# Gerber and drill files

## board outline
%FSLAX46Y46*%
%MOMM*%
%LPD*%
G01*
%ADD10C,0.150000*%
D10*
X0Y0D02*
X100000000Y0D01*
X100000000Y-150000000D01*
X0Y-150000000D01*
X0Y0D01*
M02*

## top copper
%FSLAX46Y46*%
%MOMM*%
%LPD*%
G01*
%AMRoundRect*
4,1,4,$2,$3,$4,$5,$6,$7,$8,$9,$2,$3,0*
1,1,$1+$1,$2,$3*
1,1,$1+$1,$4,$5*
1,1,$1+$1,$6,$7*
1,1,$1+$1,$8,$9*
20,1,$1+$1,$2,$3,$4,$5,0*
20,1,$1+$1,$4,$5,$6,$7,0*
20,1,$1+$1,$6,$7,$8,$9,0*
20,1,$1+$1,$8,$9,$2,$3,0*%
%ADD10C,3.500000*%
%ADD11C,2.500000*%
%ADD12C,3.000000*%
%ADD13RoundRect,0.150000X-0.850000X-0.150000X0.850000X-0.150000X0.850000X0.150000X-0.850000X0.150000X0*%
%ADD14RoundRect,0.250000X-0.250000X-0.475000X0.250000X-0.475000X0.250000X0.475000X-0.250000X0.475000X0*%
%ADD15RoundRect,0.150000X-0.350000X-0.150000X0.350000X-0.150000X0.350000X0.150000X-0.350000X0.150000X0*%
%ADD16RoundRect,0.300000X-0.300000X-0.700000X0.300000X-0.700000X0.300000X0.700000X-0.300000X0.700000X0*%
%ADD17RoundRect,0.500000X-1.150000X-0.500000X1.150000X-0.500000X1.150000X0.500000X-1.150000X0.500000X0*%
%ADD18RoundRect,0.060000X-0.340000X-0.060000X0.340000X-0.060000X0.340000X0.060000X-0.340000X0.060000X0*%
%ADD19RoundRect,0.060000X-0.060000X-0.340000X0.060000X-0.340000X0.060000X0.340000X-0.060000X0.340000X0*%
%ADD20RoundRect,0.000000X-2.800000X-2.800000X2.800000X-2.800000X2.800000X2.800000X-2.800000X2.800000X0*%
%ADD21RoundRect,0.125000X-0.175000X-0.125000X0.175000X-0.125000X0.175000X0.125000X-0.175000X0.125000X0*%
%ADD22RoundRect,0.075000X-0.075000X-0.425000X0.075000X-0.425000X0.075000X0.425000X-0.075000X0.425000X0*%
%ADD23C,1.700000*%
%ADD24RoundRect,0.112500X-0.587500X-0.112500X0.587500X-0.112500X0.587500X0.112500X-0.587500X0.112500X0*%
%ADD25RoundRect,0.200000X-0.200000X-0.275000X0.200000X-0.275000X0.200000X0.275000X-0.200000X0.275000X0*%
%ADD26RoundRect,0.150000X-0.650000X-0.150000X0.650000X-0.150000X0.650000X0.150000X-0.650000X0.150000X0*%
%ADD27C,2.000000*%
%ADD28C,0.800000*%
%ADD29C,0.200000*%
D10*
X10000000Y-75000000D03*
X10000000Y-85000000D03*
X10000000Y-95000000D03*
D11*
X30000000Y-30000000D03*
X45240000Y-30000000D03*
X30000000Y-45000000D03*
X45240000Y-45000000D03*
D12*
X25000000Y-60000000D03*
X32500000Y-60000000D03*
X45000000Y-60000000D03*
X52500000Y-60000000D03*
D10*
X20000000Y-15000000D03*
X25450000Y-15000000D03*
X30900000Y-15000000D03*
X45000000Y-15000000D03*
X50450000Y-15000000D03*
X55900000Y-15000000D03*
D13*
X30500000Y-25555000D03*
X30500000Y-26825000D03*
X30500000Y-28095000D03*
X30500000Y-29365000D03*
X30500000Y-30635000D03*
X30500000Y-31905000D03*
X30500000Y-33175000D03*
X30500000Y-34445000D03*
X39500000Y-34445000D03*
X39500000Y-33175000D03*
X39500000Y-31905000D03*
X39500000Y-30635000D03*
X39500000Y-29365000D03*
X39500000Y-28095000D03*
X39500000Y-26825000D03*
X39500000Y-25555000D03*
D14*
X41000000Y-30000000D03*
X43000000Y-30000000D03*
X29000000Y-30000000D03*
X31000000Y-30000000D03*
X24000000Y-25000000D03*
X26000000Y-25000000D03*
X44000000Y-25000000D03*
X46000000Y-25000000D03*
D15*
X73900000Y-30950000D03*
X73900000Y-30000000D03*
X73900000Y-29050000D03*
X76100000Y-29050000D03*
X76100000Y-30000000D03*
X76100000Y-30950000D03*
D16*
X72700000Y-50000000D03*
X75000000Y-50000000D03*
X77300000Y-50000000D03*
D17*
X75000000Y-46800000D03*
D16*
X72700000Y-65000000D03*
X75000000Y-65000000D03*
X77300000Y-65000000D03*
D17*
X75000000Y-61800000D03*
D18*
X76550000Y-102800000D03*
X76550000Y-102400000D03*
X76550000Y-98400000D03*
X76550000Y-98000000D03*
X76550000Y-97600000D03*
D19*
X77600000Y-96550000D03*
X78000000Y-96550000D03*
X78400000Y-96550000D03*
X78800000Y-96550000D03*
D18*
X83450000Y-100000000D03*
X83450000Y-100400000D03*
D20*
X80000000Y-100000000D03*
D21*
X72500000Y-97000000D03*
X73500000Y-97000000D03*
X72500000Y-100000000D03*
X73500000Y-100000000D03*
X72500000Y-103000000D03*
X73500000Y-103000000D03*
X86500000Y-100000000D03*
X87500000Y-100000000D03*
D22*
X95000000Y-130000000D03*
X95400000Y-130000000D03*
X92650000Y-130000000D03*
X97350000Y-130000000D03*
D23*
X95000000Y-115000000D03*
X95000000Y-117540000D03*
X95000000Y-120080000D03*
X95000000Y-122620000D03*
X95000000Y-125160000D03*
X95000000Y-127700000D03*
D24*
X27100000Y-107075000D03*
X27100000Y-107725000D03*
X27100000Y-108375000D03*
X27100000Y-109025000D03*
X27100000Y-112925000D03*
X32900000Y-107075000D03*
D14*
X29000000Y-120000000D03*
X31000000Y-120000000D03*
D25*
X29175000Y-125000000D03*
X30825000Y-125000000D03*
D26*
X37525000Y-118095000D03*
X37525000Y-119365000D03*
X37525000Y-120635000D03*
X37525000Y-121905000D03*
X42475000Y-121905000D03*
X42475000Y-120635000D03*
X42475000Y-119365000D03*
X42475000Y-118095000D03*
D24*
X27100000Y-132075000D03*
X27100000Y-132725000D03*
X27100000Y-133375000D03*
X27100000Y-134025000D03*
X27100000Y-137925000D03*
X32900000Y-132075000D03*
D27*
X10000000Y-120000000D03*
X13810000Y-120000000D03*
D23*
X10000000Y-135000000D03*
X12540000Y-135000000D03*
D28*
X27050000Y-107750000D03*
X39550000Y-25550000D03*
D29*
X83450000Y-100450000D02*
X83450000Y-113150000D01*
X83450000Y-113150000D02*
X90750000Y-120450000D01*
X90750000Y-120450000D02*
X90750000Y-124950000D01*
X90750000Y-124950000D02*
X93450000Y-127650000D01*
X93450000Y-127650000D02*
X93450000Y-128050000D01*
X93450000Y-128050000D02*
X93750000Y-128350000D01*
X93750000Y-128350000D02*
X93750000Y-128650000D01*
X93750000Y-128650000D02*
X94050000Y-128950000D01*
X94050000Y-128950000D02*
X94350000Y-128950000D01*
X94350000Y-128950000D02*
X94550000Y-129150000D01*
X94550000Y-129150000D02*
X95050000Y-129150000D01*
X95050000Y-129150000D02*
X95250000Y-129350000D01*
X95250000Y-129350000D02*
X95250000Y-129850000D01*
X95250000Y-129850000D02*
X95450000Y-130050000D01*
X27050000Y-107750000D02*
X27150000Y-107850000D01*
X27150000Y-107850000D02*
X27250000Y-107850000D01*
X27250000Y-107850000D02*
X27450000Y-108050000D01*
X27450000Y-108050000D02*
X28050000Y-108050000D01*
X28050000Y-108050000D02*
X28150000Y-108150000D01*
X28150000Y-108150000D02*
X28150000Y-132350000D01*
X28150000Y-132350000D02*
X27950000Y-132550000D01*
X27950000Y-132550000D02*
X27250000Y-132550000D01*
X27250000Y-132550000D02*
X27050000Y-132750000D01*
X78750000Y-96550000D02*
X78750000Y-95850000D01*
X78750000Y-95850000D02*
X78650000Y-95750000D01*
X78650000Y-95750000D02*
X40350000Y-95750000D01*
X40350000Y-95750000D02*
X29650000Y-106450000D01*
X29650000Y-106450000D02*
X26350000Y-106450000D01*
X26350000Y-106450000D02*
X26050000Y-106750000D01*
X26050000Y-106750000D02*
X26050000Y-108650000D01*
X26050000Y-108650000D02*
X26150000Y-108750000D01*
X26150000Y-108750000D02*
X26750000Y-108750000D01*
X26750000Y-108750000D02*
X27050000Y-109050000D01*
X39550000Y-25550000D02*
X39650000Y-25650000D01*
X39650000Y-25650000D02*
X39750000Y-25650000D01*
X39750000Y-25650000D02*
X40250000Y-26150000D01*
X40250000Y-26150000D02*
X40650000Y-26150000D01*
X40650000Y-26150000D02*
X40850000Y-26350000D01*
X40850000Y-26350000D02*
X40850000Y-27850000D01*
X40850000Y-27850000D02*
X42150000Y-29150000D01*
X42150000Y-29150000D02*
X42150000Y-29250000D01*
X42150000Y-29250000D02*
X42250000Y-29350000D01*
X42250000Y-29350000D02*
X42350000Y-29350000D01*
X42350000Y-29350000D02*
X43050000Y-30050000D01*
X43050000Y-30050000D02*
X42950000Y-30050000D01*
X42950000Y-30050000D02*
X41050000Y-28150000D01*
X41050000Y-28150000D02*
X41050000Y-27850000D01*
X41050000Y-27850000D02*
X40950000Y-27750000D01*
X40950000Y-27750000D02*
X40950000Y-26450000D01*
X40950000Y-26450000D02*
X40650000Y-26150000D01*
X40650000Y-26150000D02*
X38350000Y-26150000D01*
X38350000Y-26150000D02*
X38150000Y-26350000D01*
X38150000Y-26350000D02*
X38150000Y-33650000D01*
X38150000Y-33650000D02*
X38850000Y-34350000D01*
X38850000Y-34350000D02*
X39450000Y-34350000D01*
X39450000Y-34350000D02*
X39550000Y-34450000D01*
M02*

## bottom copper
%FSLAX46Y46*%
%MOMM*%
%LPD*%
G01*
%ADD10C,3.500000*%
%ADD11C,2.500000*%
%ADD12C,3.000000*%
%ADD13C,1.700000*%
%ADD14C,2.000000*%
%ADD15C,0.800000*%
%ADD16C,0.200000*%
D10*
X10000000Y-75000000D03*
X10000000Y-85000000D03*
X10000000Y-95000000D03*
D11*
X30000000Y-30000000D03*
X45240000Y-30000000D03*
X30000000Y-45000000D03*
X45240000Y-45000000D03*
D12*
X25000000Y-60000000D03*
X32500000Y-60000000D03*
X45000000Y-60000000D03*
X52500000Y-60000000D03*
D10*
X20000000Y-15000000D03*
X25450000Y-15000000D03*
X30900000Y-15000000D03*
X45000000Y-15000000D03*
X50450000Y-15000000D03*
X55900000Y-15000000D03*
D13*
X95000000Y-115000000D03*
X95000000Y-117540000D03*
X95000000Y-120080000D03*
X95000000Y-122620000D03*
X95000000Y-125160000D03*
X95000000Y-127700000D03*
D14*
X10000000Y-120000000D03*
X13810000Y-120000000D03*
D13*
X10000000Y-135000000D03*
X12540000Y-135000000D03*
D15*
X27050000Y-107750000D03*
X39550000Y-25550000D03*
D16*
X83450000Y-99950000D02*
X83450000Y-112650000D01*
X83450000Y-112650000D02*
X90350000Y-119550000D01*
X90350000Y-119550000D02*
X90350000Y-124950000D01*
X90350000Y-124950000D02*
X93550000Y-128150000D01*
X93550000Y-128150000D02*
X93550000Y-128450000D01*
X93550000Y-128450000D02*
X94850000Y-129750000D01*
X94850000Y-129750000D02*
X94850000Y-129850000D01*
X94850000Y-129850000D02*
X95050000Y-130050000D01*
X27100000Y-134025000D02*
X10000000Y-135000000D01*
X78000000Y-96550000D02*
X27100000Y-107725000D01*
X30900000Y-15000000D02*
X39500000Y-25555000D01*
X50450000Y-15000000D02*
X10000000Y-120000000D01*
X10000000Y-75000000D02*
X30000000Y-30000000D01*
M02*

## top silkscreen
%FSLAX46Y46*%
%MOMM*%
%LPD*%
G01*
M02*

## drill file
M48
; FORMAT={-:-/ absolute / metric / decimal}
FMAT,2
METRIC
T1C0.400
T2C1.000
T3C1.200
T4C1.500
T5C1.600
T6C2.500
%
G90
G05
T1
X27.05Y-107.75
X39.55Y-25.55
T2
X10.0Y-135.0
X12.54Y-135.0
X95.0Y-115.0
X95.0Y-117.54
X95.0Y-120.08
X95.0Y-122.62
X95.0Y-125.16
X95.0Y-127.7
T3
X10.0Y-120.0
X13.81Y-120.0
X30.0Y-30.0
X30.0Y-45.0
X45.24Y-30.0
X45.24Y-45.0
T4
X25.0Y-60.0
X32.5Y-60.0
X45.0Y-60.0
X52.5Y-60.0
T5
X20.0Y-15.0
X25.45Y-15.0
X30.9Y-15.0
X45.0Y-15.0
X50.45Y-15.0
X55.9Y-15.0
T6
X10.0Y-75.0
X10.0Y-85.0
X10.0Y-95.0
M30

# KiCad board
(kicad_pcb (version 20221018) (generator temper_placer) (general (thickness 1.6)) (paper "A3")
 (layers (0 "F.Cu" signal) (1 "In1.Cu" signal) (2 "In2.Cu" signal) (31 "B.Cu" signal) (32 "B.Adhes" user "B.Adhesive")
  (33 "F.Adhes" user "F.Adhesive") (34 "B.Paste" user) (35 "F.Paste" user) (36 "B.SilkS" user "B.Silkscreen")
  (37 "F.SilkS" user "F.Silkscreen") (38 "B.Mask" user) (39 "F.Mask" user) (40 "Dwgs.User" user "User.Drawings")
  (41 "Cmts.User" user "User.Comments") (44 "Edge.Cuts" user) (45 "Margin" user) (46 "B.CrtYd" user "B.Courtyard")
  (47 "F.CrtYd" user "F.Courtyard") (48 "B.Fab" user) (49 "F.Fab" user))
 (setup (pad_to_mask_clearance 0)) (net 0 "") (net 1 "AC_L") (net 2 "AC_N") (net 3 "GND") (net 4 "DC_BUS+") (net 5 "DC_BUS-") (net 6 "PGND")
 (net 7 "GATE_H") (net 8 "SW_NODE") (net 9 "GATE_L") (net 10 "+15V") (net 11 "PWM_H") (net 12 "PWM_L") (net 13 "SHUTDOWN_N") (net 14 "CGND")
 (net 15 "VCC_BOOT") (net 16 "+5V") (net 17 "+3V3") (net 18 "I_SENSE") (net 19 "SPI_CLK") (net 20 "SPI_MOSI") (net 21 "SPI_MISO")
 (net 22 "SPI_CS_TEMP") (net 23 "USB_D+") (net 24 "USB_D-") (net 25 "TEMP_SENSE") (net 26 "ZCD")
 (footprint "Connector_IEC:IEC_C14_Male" (layer "F.Cu") (at 10 75) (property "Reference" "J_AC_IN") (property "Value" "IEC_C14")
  (pad "1" thru_hole circle (at 0 0) (size 3.5 3.5) (drill 2.5) (layers *.Cu *.Mask) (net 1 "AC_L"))
  (pad "2" thru_hole circle (at 0 10) (size 3.5 3.5) (drill 2.5) (layers *.Cu *.Mask) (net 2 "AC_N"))
  (pad "3" thru_hole circle (at 0 20) (size 3.5 3.5) (drill 2.5) (layers *.Cu *.Mask) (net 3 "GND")))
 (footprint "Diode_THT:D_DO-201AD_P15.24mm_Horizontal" (layer "F.Cu") (at 30 30) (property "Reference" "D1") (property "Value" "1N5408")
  (pad "1" thru_hole circle (at 0 0) (size 2.5 2.5) (drill 1.2) (layers *.Cu *.Mask) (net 1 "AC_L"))
  (pad "2" thru_hole circle (at 15.24 0) (size 2.5 2.5) (drill 1.2) (layers *.Cu *.Mask) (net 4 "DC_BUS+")))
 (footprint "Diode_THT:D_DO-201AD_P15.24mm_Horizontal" (layer "F.Cu") (at 30 45) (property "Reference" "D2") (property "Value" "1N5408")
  (pad "1" thru_hole circle (at 0 0) (size 2.5 2.5) (drill 1.2) (layers *.Cu *.Mask) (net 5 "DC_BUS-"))
  (pad "2" thru_hole circle (at 15.24 0) (size 2.5 2.5) (drill 1.2) (layers *.Cu *.Mask) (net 2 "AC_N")))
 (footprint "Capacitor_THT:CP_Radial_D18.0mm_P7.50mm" (layer "F.Cu") (at 25 60) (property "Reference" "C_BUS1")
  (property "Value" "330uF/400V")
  (pad "1" thru_hole circle (at 0 0) (size 3 3) (drill 1.5) (layers *.Cu *.Mask) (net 4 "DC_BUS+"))
  (pad "2" thru_hole circle (at 7.5 0) (size 3 3) (drill 1.5) (layers *.Cu *.Mask) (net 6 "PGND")))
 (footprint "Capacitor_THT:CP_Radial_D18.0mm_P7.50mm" (layer "F.Cu") (at 45 60) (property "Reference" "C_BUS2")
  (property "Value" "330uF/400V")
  (pad "1" thru_hole circle (at 0 0) (size 3 3) (drill 1.5) (layers *.Cu *.Mask) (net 6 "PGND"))
  (pad "2" thru_hole circle (at 7.5 0) (size 3 3) (drill 1.5) (layers *.Cu *.Mask) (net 5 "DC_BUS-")))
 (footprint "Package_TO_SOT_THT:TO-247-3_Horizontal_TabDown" (layer "F.Cu") (at 20 15) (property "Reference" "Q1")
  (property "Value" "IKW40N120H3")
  (pad "1" thru_hole circle (at 0 0) (size 3.5 3.5) (drill 1.6) (layers *.Cu *.Mask) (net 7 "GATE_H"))
  (pad "2" thru_hole circle (at 5.45 0) (size 3.5 3.5) (drill 1.6) (layers *.Cu *.Mask) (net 4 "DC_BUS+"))
  (pad "3" thru_hole circle (at 10.9 0) (size 3.5 3.5) (drill 1.6) (layers *.Cu *.Mask) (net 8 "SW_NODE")))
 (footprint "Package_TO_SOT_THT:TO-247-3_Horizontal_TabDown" (layer "F.Cu") (at 45 15) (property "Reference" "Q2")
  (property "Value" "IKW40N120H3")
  (pad "1" thru_hole circle (at 0 0) (size 3.5 3.5) (drill 1.6) (layers *.Cu *.Mask) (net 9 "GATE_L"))
  (pad "2" thru_hole circle (at 5.45 0) (size 3.5 3.5) (drill 1.6) (layers *.Cu *.Mask) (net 8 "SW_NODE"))
  (pad "3" thru_hole circle (at 10.9 0) (size 3.5 3.5) (drill 1.6) (layers *.Cu *.Mask) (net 5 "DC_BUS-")))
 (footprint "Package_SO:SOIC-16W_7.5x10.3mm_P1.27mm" (layer "F.Cu") (at 35 30) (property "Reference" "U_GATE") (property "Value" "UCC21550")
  (pad "1" smd roundrect (at -4.5 -4.445) (size 2 0.6) (layers "F.Cu" "F.Paste" "F.Mask") (roundrect_rratio 0.25) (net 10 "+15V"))
  (pad "2" smd roundrect (at -4.5 -3.175) (size 2 0.6) (layers "F.Cu" "F.Paste" "F.Mask") (roundrect_rratio 0.25) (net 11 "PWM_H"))
  (pad "3" smd roundrect (at -4.5 -1.905) (size 2 0.6) (layers "F.Cu" "F.Paste" "F.Mask") (roundrect_rratio 0.25) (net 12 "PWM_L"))
  (pad "4" smd roundrect (at -4.5 -0.635) (size 2 0.6) (layers "F.Cu" "F.Paste" "F.Mask") (roundrect_rratio 0.25) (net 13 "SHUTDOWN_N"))
  (pad "5" smd roundrect (at -4.5 0.635) (size 2 0.6) (layers "F.Cu" "F.Paste" "F.Mask") (roundrect_rratio 0.25) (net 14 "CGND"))
  (pad "6" smd roundrect (at -4.5 1.905) (size 2 0.6) (layers "F.Cu" "F.Paste" "F.Mask") (roundrect_rratio 0.25) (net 14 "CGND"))
  (pad "7" smd roundrect (at -4.5 3.175) (size 2 0.6) (layers "F.Cu" "F.Paste" "F.Mask") (roundrect_rratio 0.25) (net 14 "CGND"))
  (pad "8" smd roundrect (at -4.5 4.445) (size 2 0.6) (layers "F.Cu" "F.Paste" "F.Mask") (roundrect_rratio 0.25) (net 14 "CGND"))
  (pad "9" smd roundrect (at 4.5 4.445) (size 2 0.6) (layers "F.Cu" "F.Paste" "F.Mask") (roundrect_rratio 0.25) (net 8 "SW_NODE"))
  (pad "10" smd roundrect (at 4.5 3.175) (size 2 0.6) (layers "F.Cu" "F.Paste" "F.Mask") (roundrect_rratio 0.25) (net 9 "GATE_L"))
  (pad "11" smd roundrect (at 4.5 1.905) (size 2 0.6) (layers "F.Cu" "F.Paste" "F.Mask") (roundrect_rratio 0.25) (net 10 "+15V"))
  (pad "12" smd roundrect (at 4.5 0.635) (size 2 0.6) (layers "F.Cu" "F.Paste" "F.Mask") (roundrect_rratio 0.25) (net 6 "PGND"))
  (pad "13" smd roundrect (at 4.5 -0.635) (size 2 0.6) (layers "F.Cu" "F.Paste" "F.Mask") (roundrect_rratio 0.25) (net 6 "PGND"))
  (pad "14" smd roundrect (at 4.5 -1.905) (size 2 0.6) (layers "F.Cu" "F.Paste" "F.Mask") (roundrect_rratio 0.25) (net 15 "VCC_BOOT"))
  (pad "15" smd roundrect (at 4.5 -3.175) (size 2 0.6) (layers "F.Cu" "F.Paste" "F.Mask") (roundrect_rratio 0.25) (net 7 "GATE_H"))
  (pad "16" smd roundrect (at 4.5 -4.445) (size 2 0.6) (layers "F.Cu" "F.Paste" "F.Mask") (roundrect_rratio 0.25) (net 8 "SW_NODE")))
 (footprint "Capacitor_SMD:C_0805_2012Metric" (layer "F.Cu") (at 42 30) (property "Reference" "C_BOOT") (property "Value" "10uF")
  (pad "1" smd roundrect (at -1 0) (size 1 1.45) (layers "F.Cu" "F.Paste" "F.Mask") (roundrect_rratio 0.25) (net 15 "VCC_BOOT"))
  (pad "2" smd roundrect (at 1 0) (size 1 1.45) (layers "F.Cu" "F.Paste" "F.Mask") (roundrect_rratio 0.25) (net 8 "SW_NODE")))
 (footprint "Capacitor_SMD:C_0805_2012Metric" (layer "F.Cu") (at 30 30) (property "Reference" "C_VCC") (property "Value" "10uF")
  (pad "1" smd roundrect (at -1 0) (size 1 1.45) (layers "F.Cu" "F.Paste" "F.Mask") (roundrect_rratio 0.25) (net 10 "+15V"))
  (pad "2" smd roundrect (at 1 0) (size 1 1.45) (layers "F.Cu" "F.Paste" "F.Mask") (roundrect_rratio 0.25) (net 14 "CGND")))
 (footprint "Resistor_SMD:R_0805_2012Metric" (layer "F.Cu") (at 25 25) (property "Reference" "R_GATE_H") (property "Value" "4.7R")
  (pad "1" smd roundrect (at -1 0) (size 1 1.45) (layers "F.Cu" "F.Paste" "F.Mask") (roundrect_rratio 0.25) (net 7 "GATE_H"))
  (pad "2" smd roundrect (at 1 0) (size 1 1.45) (layers "F.Cu" "F.Paste" "F.Mask") (roundrect_rratio 0.25) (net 7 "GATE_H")))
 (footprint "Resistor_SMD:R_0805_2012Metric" (layer "F.Cu") (at 45 25) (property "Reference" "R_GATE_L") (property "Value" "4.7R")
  (pad "1" smd roundrect (at -1 0) (size 1 1.45) (layers "F.Cu" "F.Paste" "F.Mask") (roundrect_rratio 0.25) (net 9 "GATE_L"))
  (pad "2" smd roundrect (at 1 0) (size 1 1.45) (layers "F.Cu" "F.Paste" "F.Mask") (roundrect_rratio 0.25) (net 9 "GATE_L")))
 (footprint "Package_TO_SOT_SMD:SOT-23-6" (layer "F.Cu") (at 75 30) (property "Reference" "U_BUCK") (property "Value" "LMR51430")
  (pad "1" smd roundrect (at -1.1 0.95) (size 1 0.6) (layers "F.Cu" "F.Paste" "F.Mask") (roundrect_rratio 0.25) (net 3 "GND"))
  (pad "2" smd roundrect (at -1.1 0) (size 1 0.6) (layers "F.Cu" "F.Paste" "F.Mask") (roundrect_rratio 0.25) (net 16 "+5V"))
  (pad "3" smd roundrect (at -1.1 -0.95) (size 1 0.6) (layers "F.Cu" "F.Paste" "F.Mask") (roundrect_rratio 0.25) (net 10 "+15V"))
  (pad "4" smd roundrect (at 1.1 -0.95) (size 1 0.6) (layers "F.Cu" "F.Paste" "F.Mask") (roundrect_rratio 0.25) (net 16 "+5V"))
  (pad "5" smd roundrect (at 1.1 0) (size 1 0.6) (layers "F.Cu" "F.Paste" "F.Mask") (roundrect_rratio 0.25) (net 3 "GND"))
  (pad "6" smd roundrect (at 1.1 0.95) (size 1 0.6) (layers "F.Cu" "F.Paste" "F.Mask") (roundrect_rratio 0.25) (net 3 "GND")))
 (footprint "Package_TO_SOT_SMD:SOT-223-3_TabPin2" (layer "F.Cu") (at 75 50) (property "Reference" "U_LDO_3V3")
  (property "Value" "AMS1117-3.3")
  (pad "1" smd roundrect (at -2.3 0) (size 1.2 2) (layers "F.Cu" "F.Paste" "F.Mask") (roundrect_rratio 0.25) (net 3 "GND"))
  (pad "2" smd roundrect (at 0 0) (size 1.2 2) (layers "F.Cu" "F.Paste" "F.Mask") (roundrect_rratio 0.25) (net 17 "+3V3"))
  (pad "3" smd roundrect (at 2.3 0) (size 1.2 2) (layers "F.Cu" "F.Paste" "F.Mask") (roundrect_rratio 0.25) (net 16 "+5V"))
  (pad "4" smd roundrect (at 0 -3.2) (size 3.3 2) (layers "F.Cu" "F.Paste" "F.Mask") (roundrect_rratio 0.25) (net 17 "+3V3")))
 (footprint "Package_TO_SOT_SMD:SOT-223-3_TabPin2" (layer "F.Cu") (at 75 65) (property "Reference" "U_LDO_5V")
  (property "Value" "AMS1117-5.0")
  (pad "1" smd roundrect (at -2.3 0) (size 1.2 2) (layers "F.Cu" "F.Paste" "F.Mask") (roundrect_rratio 0.25) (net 3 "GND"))
  (pad "2" smd roundrect (at 0 0) (size 1.2 2) (layers "F.Cu" "F.Paste" "F.Mask") (roundrect_rratio 0.25) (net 16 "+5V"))
  (pad "3" smd roundrect (at 2.3 0) (size 1.2 2) (layers "F.Cu" "F.Paste" "F.Mask") (roundrect_rratio 0.25) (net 10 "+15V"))
  (pad "4" smd roundrect (at 0 -3.2) (size 3.3 2) (layers "F.Cu" "F.Paste" "F.Mask") (roundrect_rratio 0.25) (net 16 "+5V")))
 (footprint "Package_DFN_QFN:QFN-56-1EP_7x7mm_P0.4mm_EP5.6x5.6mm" (layer "F.Cu") (at 80 100) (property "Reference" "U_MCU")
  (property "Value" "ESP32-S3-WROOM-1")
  (pad "1" smd roundrect (at -3.45 2.8) (size 0.8 0.24) (layers "F.Cu" "F.Paste" "F.Mask") (roundrect_rratio 0.25) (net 17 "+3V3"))
  (pad "2" smd roundrect (at -3.45 2.4) (size 0.8 0.24) (layers "F.Cu" "F.Paste" "F.Mask") (roundrect_rratio 0.25) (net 3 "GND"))
  (pad "13" smd roundrect (at -3.45 -1.6) (size 0.8 0.24) (layers "F.Cu" "F.Paste" "F.Mask") (roundrect_rratio 0.25) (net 11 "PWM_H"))
  (pad "14" smd roundrect (at -3.45 -2) (size 0.8 0.24) (layers "F.Cu" "F.Paste" "F.Mask") (roundrect_rratio 0.25) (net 12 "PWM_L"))
  (pad "15" smd roundrect (at -3.45 -2.4) (size 0.8 0.24) (layers "F.Cu" "F.Paste" "F.Mask") (roundrect_rratio 0.25) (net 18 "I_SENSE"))
  (pad "20" smd roundrect (at -2.4 -3.45) (size 0.24 0.8) (layers "F.Cu" "F.Paste" "F.Mask") (roundrect_rratio 0.25) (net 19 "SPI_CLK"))
  (pad "21" smd roundrect (at -2 -3.45) (size 0.24 0.8) (layers "F.Cu" "F.Paste" "F.Mask") (roundrect_rratio 0.25) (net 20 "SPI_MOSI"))
  (pad "22" smd roundrect (at -1.6 -3.45) (size 0.24 0.8) (layers "F.Cu" "F.Paste" "F.Mask") (roundrect_rratio 0.25) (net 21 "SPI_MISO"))
  (pad "23" smd roundrect (at -1.2 -3.45) (size 0.24 0.8) (layers "F.Cu" "F.Paste" "F.Mask") (roundrect_rratio 0.25) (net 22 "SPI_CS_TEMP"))
  (pad "40" smd roundrect (at 3.45 0) (size 0.8 0.24) (layers "F.Cu" "F.Paste" "F.Mask") (roundrect_rratio 0.25) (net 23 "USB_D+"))
  (pad "41" smd roundrect (at 3.45 0.4) (size 0.8 0.24) (layers "F.Cu" "F.Paste" "F.Mask") (roundrect_rratio 0.25) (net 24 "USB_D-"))
  (pad "57" smd roundrect (at 0 0) (size 5.6 5.6) (layers "F.Cu" "F.Paste" "F.Mask") (roundrect_rratio 0) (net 3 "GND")))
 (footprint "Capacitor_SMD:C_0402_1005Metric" (layer "F.Cu") (at 73 97) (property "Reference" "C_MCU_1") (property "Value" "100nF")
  (pad "1" smd roundrect (at -0.5 0) (size 0.6 0.5) (layers "F.Cu" "F.Paste" "F.Mask") (roundrect_rratio 0.25) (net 17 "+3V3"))
  (pad "2" smd roundrect (at 0.5 0) (size 0.6 0.5) (layers "F.Cu" "F.Paste" "F.Mask") (roundrect_rratio 0.25) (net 3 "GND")))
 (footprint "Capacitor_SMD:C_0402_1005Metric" (layer "F.Cu") (at 73 100) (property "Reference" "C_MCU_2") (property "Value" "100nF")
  (pad "1" smd roundrect (at -0.5 0) (size 0.6 0.5) (layers "F.Cu" "F.Paste" "F.Mask") (roundrect_rratio 0.25) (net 17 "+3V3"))
  (pad "2" smd roundrect (at 0.5 0) (size 0.6 0.5) (layers "F.Cu" "F.Paste" "F.Mask") (roundrect_rratio 0.25) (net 3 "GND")))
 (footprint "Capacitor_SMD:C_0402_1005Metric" (layer "F.Cu") (at 73 103) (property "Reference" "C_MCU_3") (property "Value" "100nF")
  (pad "1" smd roundrect (at -0.5 0) (size 0.6 0.5) (layers "F.Cu" "F.Paste" "F.Mask") (roundrect_rratio 0.25) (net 17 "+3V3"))
  (pad "2" smd roundrect (at 0.5 0) (size 0.6 0.5) (layers "F.Cu" "F.Paste" "F.Mask") (roundrect_rratio 0.25) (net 3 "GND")))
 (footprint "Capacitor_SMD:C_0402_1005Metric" (layer "F.Cu") (at 87 100) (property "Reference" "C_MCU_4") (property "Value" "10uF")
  (pad "1" smd roundrect (at -0.5 0) (size 0.6 0.5) (layers "F.Cu" "F.Paste" "F.Mask") (roundrect_rratio 0.25) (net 17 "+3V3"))
  (pad "2" smd roundrect (at 0.5 0) (size 0.6 0.5) (layers "F.Cu" "F.Paste" "F.Mask") (roundrect_rratio 0.25) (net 3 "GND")))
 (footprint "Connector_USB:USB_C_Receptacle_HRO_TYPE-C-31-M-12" (layer "F.Cu") (at 95 130) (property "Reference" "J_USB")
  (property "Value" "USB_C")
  (pad "A6" smd roundrect (at 0 0) (size 0.3 1) (layers "F.Cu" "F.Paste" "F.Mask") (roundrect_rratio 0.25) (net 23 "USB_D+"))
  (pad "B6" smd roundrect (at 0.4 0) (size 0.3 1) (layers "F.Cu" "F.Paste" "F.Mask") (roundrect_rratio 0.25) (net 24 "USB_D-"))
  (pad "A1" smd roundrect (at -2.35 0) (size 0.3 1) (layers "F.Cu" "F.Paste" "F.Mask") (roundrect_rratio 0.25) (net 3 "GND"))
  (pad "A12" smd roundrect (at 2.35 0) (size 0.3 1) (layers "F.Cu" "F.Paste" "F.Mask") (roundrect_rratio 0.25) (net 3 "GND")))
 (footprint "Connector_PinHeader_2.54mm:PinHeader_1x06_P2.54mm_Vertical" (layer "F.Cu") (at 95 115) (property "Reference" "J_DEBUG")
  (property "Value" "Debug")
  (pad "1" thru_hole circle (at 0 0) (size 1.7 1.7) (drill 1) (layers *.Cu *.Mask) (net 3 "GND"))
  (pad "2" thru_hole circle (at 0 2.54) (size 1.7 1.7) (drill 1) (layers *.Cu *.Mask) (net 17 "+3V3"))
  (pad "3" thru_hole circle (at 0 5.08) (size 1.7 1.7) (drill 1) (layers *.Cu *.Mask) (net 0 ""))
  (pad "4" thru_hole circle (at 0 7.62) (size 1.7 1.7) (drill 1) (layers *.Cu *.Mask) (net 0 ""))
  (pad "5" thru_hole circle (at 0 10.16) (size 1.7 1.7) (drill 1) (layers *.Cu *.Mask) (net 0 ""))
  (pad "6" thru_hole circle (at 0 12.7) (size 1.7 1.7) (drill 1) (layers *.Cu *.Mask) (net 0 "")))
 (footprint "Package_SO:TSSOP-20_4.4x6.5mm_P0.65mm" (layer "F.Cu") (at 30 110) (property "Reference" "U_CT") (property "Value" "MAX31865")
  (pad "1" smd roundrect (at -2.9 -2.925) (size 1.4 0.45) (layers "F.Cu" "F.Paste" "F.Mask") (roundrect_rratio 0.25) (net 19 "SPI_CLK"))
  (pad "2" smd roundrect (at -2.9 -2.275) (size 1.4 0.45) (layers "F.Cu" "F.Paste" "F.Mask") (roundrect_rratio 0.25) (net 20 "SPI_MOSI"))
  (pad "3" smd roundrect (at -2.9 -1.625) (size 1.4 0.45) (layers "F.Cu" "F.Paste" "F.Mask") (roundrect_rratio 0.25) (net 21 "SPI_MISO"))
  (pad "4" smd roundrect (at -2.9 -0.975) (size 1.4 0.45) (layers "F.Cu" "F.Paste" "F.Mask") (roundrect_rratio 0.25) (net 22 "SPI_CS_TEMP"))
  (pad "10" smd roundrect (at -2.9 2.925) (size 1.4 0.45) (layers "F.Cu" "F.Paste" "F.Mask") (roundrect_rratio 0.25) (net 3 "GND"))
  (pad "20" smd roundrect (at 2.9 -2.925) (size 1.4 0.45) (layers "F.Cu" "F.Paste" "F.Mask") (roundrect_rratio 0.25) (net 17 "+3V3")))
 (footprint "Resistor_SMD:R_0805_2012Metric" (layer "F.Cu") (at 30 120) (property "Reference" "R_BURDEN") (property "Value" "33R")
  (pad "1" smd roundrect (at -1 0) (size 1 1.45) (layers "F.Cu" "F.Paste" "F.Mask") (roundrect_rratio 0.25) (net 18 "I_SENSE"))
  (pad "2" smd roundrect (at 1 0) (size 1 1.45) (layers "F.Cu" "F.Paste" "F.Mask") (roundrect_rratio 0.25) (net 3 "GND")))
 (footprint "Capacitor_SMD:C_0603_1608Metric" (layer "F.Cu") (at 30 125) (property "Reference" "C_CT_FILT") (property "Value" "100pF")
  (pad "1" smd roundrect (at -0.825 0) (size 0.8 0.95) (layers "F.Cu" "F.Paste" "F.Mask") (roundrect_rratio 0.25) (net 18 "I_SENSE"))
  (pad "2" smd roundrect (at 0.825 0) (size 0.8 0.95) (layers "F.Cu" "F.Paste" "F.Mask") (roundrect_rratio 0.25) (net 3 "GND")))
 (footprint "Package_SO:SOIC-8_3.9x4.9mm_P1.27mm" (layer "F.Cu") (at 40 120) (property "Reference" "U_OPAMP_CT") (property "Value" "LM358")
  (pad "1" smd roundrect (at -2.475 -1.905) (size 1.6 0.6) (layers "F.Cu" "F.Paste" "F.Mask") (roundrect_rratio 0.25) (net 18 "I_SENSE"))
  (pad "2" smd roundrect (at -2.475 -0.635) (size 1.6 0.6) (layers "F.Cu" "F.Paste" "F.Mask") (roundrect_rratio 0.25) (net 18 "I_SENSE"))
  (pad "3" smd roundrect (at -2.475 0.635) (size 1.6 0.6) (layers "F.Cu" "F.Paste" "F.Mask") (roundrect_rratio 0.25) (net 18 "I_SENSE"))
  (pad "4" smd roundrect (at -2.475 1.905) (size 1.6 0.6) (layers "F.Cu" "F.Paste" "F.Mask") (roundrect_rratio 0.25) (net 3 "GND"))
  (pad "5" smd roundrect (at 2.475 1.905) (size 1.6 0.6) (layers "F.Cu" "F.Paste" "F.Mask") (roundrect_rratio 0.25) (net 18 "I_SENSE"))
  (pad "6" smd roundrect (at 2.475 0.635) (size 1.6 0.6) (layers "F.Cu" "F.Paste" "F.Mask") (roundrect_rratio 0.25) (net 18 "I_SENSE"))
  (pad "7" smd roundrect (at 2.475 -0.635) (size 1.6 0.6) (layers "F.Cu" "F.Paste" "F.Mask") (roundrect_rratio 0.25) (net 16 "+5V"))
  (pad "8" smd roundrect (at 2.475 -1.905) (size 1.6 0.6) (layers "F.Cu" "F.Paste" "F.Mask") (roundrect_rratio 0.25) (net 16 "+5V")))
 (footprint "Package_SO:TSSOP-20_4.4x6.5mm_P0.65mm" (layer "F.Cu") (at 30 135) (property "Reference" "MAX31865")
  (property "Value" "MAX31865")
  (pad "1" smd roundrect (at -2.9 -2.925) (size 1.4 0.45) (layers "F.Cu" "F.Paste" "F.Mask") (roundrect_rratio 0.25) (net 19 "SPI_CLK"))
  (pad "2" smd roundrect (at -2.9 -2.275) (size 1.4 0.45) (layers "F.Cu" "F.Paste" "F.Mask") (roundrect_rratio 0.25) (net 20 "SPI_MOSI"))
  (pad "3" smd roundrect (at -2.9 -1.625) (size 1.4 0.45) (layers "F.Cu" "F.Paste" "F.Mask") (roundrect_rratio 0.25) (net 21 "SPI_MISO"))
  (pad "4" smd roundrect (at -2.9 -0.975) (size 1.4 0.45) (layers "F.Cu" "F.Paste" "F.Mask") (roundrect_rratio 0.25) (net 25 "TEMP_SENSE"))
  (pad "10" smd roundrect (at -2.9 2.925) (size 1.4 0.45) (layers "F.Cu" "F.Paste" "F.Mask") (roundrect_rratio 0.25) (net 3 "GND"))
  (pad "20" smd roundrect (at 2.9 -2.925) (size 1.4 0.45) (layers "F.Cu" "F.Paste" "F.Mask") (roundrect_rratio 0.25) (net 17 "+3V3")))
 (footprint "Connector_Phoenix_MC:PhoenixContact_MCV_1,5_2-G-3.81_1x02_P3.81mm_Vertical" (layer "F.Cu") (at 10 120)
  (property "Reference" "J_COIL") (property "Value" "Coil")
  (pad "1" thru_hole circle (at 0 0) (size 2 2) (drill 1.2) (layers *.Cu *.Mask) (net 8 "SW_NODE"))
  (pad "2" thru_hole circle (at 3.81 0) (size 2 2) (drill 1.2) (layers *.Cu *.Mask) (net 3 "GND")))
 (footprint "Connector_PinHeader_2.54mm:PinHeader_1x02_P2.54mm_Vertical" (layer "F.Cu") (at 10 135) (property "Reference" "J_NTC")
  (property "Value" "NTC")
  (pad "1" thru_hole circle (at 0 0) (size 1.7 1.7) (drill 1) (layers *.Cu *.Mask) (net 25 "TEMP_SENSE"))
  (pad "2" thru_hole circle (at 2.54 0) (size 1.7 1.7) (drill 1) (layers *.Cu *.Mask) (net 3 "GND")))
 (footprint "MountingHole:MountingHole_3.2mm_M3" (layer "F.Cu") (at 5 5) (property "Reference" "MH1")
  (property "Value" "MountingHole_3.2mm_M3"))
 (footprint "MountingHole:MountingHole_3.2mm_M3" (layer "F.Cu") (at 95 5) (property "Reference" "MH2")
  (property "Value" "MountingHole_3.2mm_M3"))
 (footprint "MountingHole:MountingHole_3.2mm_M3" (layer "F.Cu") (at 5 145) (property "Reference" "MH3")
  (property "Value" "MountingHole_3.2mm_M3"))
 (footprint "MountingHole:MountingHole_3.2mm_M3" (layer "F.Cu") (at 95 145) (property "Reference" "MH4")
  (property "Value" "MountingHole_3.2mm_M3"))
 (gr_rect (start 0 0) (end 100 150) (layer "Edge.Cuts") (width 0.15))
 (segment (start 83.45 99.95) (end 83.45 112.65) (width 0.2) (layer "B.Cu") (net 23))
 (segment (start 83.45 112.65) (end 90.35000000000001 119.55000000000001) (width 0.2) (layer "B.Cu") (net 23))
 (segment (start 90.35000000000001 119.55000000000001) (end 90.35000000000001 124.95) (width 0.2) (layer "B.Cu") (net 23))
 (segment (start 90.35000000000001 124.95) (end 93.55000000000001 128.15) (width 0.2) (layer "B.Cu") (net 23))
 (segment (start 93.55000000000001 128.15) (end 93.55000000000001 128.45000000000002) (width 0.2) (layer "B.Cu") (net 23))
 (segment (start 93.55000000000001 128.45000000000002) (end 94.85000000000001 129.75) (width 0.2) (layer "B.Cu") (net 23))
 (segment (start 94.85000000000001 129.75) (end 94.85000000000001 129.85) (width 0.2) (layer "B.Cu") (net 23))
 (segment (start 94.85000000000001 129.85) (end 95.05000000000001 130.05) (width 0.2) (layer "B.Cu") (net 23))
 (segment (start 27.09999990463257 134.02499997615814) (end 10.000000019073486 135.0) (width 0.2) (layer "B.Cu") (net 25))
 (segment (start 83.45 100.45) (end 83.45 113.15) (width 0.2) (layer "F.Cu") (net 24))
 (segment (start 83.45 113.15) (end 90.75 120.45) (width 0.2) (layer "F.Cu") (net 24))
 (segment (start 90.75 120.45) (end 90.75 124.95) (width 0.2) (layer "F.Cu") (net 24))
 (segment (start 90.75 124.95) (end 93.45 127.65) (width 0.2) (layer "F.Cu") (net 24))
 (segment (start 93.45 127.65) (end 93.45 128.05) (width 0.2) (layer "F.Cu") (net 24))
 (segment (start 93.45 128.05) (end 93.75 128.35) (width 0.2) (layer "F.Cu") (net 24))
 (segment (start 93.75 128.35) (end 93.75 128.65) (width 0.2) (layer "F.Cu") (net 24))
 (segment (start 93.75 128.65) (end 94.05000000000001 128.95000000000002) (width 0.2) (layer "F.Cu") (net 24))
 (segment (start 94.05000000000001 128.95000000000002) (end 94.35000000000001 128.95000000000002) (width 0.2) (layer "F.Cu") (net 24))
 (segment (start 94.35000000000001 128.95000000000002) (end 94.55000000000001 129.15) (width 0.2) (layer "F.Cu") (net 24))
 (segment (start 94.55000000000001 129.15) (end 95.05000000000001 129.15) (width 0.2) (layer "F.Cu") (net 24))
 (segment (start 95.05000000000001 129.15) (end 95.25 129.35) (width 0.2) (layer "F.Cu") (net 24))
 (segment (start 95.25 129.35) (end 95.25 129.85) (width 0.2) (layer "F.Cu") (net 24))
 (segment (start 95.25 129.85) (end 95.45 130.05) (width 0.2) (layer "F.Cu") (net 24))
 (segment (start 78.0 96.55) (end 27.09999990463257 107.72499990463257) (width 0.2) (layer "B.Cu") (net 20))
 (segment (start 27.05 107.75) (end 27.150000000000002 107.85000000000001) (width 0.2) (layer "F.Cu") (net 20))
 (segment (start 27.150000000000002 107.85000000000001) (end 27.25 107.85000000000001) (width 0.2) (layer "F.Cu") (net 20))
 (segment (start 27.25 107.85000000000001) (end 27.450000000000003 108.05000000000001) (width 0.2) (layer "F.Cu") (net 20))
 (segment (start 27.450000000000003 108.05000000000001) (end 28.05 108.05000000000001) (width 0.2) (layer "F.Cu") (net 20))
 (segment (start 28.05 108.05000000000001) (end 28.150000000000002 108.15) (width 0.2) (layer "F.Cu") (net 20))
 (segment (start 28.150000000000002 108.15) (end 28.150000000000002 132.35) (width 0.2) (layer "F.Cu") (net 20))
 (segment (start 28.150000000000002 132.35) (end 27.950000000000003 132.55) (width 0.2) (layer "F.Cu") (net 20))
 (segment (start 27.950000000000003 132.55) (end 27.25 132.55) (width 0.2) (layer "F.Cu") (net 20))
 (segment (start 27.25 132.55) (end 27.05 132.75) (width 0.2) (layer "F.Cu") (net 20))
 (via (at 27.05 107.75) (size 0.8) (drill 0.4) (layers "F.Cu" "B.Cu") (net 20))
 (segment (start 78.75 96.55000000000001) (end 78.75 95.85000000000001) (width 0.2) (layer "F.Cu") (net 22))
 (segment (start 78.75 95.85000000000001) (end 78.65 95.75) (width 0.2) (layer "F.Cu") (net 22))
 (segment (start 78.65 95.75) (end 40.35 95.75) (width 0.2) (layer "F.Cu") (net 22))
 (segment (start 40.35 95.75) (end 29.650000000000002 106.45) (width 0.2) (layer "F.Cu") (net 22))
 (segment (start 29.650000000000002 106.45) (end 26.35 106.45) (width 0.2) (layer "F.Cu") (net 22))
 (segment (start 26.35 106.45) (end 26.05 106.75) (width 0.2) (layer "F.Cu") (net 22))
 (segment (start 26.05 106.75) (end 26.05 108.65) (width 0.2) (layer "F.Cu") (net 22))
 (segment (start 26.05 108.65) (end 26.150000000000002 108.75) (width 0.2) (layer "F.Cu") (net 22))
 (segment (start 26.150000000000002 108.75) (end 26.75 108.75) (width 0.2) (layer "F.Cu") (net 22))
 (segment (start 26.75 108.75) (end 27.05 109.05000000000001) (width 0.2) (layer "F.Cu") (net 22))
 (segment (start 30.89999980926514 15.0) (end 39.5 25.554999828338623) (width 0.2) (layer "B.Cu") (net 8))
 (segment (start 39.550000000000004 25.55) (end 39.650000000000006 25.650000000000002) (width 0.2) (layer "F.Cu") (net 8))
 (segment (start 39.650000000000006 25.650000000000002) (end 39.75 25.650000000000002) (width 0.2) (layer "F.Cu") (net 8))
 (segment (start 39.75 25.650000000000002) (end 40.25 26.150000000000002) (width 0.2) (layer "F.Cu") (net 8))
 (segment (start 40.25 26.150000000000002) (end 40.650000000000006 26.150000000000002) (width 0.2) (layer "F.Cu") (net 8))
 (segment (start 40.650000000000006 26.150000000000002) (end 40.85 26.35) (width 0.2) (layer "F.Cu") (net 8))
 (segment (start 40.85 26.35) (end 40.85 27.85) (width 0.2) (layer "F.Cu") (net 8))
 (segment (start 40.85 27.85) (end 42.150000000000006 29.150000000000002) (width 0.2) (layer "F.Cu") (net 8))
 (segment (start 42.150000000000006 29.150000000000002) (end 42.150000000000006 29.25) (width 0.2) (layer "F.Cu") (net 8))
 (segment (start 42.150000000000006 29.25) (end 42.25 29.35) (width 0.2) (layer "F.Cu") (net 8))
 (segment (start 42.25 29.35) (end 42.35 29.35) (width 0.2) (layer "F.Cu") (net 8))
 (segment (start 42.35 29.35) (end 43.050000000000004 30.050000000000004) (width 0.2) (layer "F.Cu") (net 8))
 (segment (start 43.050000000000004 30.050000000000004) (end 42.95 30.050000000000004) (width 0.2) (layer "F.Cu") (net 8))
 (segment (start 42.95 30.050000000000004) (end 41.050000000000004 28.150000000000002) (width 0.2) (layer "F.Cu") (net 8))
 (segment (start 41.050000000000004 28.150000000000002) (end 41.050000000000004 27.85) (width 0.2) (layer "F.Cu") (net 8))
 (segment (start 41.050000000000004 27.85) (end 40.95 27.75) (width 0.2) (layer "F.Cu") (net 8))
 (segment (start 40.95 27.75) (end 40.95 26.450000000000003) (width 0.2) (layer "F.Cu") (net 8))
 (segment (start 40.95 26.450000000000003) (end 40.650000000000006 26.150000000000002) (width 0.2) (layer "F.Cu") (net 8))
 (segment (start 40.650000000000006 26.150000000000002) (end 38.35 26.150000000000002) (width 0.2) (layer "F.Cu") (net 8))
 (segment (start 38.35 26.150000000000002) (end 38.150000000000006 26.35) (width 0.2) (layer "F.Cu") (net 8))
 (segment (start 38.150000000000006 26.35) (end 38.150000000000006 33.65) (width 0.2) (layer "F.Cu") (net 8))
 (segment (start 38.150000000000006 33.65) (end 38.85 34.35) (width 0.2) (layer "F.Cu") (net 8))
 (segment (start 38.85 34.35) (end 39.45 34.35) (width 0.2) (layer "F.Cu") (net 8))
 (segment (start 39.45 34.35) (end 39.550000000000004 34.45) (width 0.2) (layer "F.Cu") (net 8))
 (segment (start 50.45 15.000000000000002) (end 10.000000028610229 120.0) (width 0.2) (layer "B.Cu") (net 8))
 (via (at 39.550000000000004 25.55) (size 0.8) (drill 0.4) (layers "F.Cu" "B.Cu") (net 8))
 (segment (start 10.0 75.0) (end 30.000000114440915 30.0) (width 0.2) (layer "B.Cu") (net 1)))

